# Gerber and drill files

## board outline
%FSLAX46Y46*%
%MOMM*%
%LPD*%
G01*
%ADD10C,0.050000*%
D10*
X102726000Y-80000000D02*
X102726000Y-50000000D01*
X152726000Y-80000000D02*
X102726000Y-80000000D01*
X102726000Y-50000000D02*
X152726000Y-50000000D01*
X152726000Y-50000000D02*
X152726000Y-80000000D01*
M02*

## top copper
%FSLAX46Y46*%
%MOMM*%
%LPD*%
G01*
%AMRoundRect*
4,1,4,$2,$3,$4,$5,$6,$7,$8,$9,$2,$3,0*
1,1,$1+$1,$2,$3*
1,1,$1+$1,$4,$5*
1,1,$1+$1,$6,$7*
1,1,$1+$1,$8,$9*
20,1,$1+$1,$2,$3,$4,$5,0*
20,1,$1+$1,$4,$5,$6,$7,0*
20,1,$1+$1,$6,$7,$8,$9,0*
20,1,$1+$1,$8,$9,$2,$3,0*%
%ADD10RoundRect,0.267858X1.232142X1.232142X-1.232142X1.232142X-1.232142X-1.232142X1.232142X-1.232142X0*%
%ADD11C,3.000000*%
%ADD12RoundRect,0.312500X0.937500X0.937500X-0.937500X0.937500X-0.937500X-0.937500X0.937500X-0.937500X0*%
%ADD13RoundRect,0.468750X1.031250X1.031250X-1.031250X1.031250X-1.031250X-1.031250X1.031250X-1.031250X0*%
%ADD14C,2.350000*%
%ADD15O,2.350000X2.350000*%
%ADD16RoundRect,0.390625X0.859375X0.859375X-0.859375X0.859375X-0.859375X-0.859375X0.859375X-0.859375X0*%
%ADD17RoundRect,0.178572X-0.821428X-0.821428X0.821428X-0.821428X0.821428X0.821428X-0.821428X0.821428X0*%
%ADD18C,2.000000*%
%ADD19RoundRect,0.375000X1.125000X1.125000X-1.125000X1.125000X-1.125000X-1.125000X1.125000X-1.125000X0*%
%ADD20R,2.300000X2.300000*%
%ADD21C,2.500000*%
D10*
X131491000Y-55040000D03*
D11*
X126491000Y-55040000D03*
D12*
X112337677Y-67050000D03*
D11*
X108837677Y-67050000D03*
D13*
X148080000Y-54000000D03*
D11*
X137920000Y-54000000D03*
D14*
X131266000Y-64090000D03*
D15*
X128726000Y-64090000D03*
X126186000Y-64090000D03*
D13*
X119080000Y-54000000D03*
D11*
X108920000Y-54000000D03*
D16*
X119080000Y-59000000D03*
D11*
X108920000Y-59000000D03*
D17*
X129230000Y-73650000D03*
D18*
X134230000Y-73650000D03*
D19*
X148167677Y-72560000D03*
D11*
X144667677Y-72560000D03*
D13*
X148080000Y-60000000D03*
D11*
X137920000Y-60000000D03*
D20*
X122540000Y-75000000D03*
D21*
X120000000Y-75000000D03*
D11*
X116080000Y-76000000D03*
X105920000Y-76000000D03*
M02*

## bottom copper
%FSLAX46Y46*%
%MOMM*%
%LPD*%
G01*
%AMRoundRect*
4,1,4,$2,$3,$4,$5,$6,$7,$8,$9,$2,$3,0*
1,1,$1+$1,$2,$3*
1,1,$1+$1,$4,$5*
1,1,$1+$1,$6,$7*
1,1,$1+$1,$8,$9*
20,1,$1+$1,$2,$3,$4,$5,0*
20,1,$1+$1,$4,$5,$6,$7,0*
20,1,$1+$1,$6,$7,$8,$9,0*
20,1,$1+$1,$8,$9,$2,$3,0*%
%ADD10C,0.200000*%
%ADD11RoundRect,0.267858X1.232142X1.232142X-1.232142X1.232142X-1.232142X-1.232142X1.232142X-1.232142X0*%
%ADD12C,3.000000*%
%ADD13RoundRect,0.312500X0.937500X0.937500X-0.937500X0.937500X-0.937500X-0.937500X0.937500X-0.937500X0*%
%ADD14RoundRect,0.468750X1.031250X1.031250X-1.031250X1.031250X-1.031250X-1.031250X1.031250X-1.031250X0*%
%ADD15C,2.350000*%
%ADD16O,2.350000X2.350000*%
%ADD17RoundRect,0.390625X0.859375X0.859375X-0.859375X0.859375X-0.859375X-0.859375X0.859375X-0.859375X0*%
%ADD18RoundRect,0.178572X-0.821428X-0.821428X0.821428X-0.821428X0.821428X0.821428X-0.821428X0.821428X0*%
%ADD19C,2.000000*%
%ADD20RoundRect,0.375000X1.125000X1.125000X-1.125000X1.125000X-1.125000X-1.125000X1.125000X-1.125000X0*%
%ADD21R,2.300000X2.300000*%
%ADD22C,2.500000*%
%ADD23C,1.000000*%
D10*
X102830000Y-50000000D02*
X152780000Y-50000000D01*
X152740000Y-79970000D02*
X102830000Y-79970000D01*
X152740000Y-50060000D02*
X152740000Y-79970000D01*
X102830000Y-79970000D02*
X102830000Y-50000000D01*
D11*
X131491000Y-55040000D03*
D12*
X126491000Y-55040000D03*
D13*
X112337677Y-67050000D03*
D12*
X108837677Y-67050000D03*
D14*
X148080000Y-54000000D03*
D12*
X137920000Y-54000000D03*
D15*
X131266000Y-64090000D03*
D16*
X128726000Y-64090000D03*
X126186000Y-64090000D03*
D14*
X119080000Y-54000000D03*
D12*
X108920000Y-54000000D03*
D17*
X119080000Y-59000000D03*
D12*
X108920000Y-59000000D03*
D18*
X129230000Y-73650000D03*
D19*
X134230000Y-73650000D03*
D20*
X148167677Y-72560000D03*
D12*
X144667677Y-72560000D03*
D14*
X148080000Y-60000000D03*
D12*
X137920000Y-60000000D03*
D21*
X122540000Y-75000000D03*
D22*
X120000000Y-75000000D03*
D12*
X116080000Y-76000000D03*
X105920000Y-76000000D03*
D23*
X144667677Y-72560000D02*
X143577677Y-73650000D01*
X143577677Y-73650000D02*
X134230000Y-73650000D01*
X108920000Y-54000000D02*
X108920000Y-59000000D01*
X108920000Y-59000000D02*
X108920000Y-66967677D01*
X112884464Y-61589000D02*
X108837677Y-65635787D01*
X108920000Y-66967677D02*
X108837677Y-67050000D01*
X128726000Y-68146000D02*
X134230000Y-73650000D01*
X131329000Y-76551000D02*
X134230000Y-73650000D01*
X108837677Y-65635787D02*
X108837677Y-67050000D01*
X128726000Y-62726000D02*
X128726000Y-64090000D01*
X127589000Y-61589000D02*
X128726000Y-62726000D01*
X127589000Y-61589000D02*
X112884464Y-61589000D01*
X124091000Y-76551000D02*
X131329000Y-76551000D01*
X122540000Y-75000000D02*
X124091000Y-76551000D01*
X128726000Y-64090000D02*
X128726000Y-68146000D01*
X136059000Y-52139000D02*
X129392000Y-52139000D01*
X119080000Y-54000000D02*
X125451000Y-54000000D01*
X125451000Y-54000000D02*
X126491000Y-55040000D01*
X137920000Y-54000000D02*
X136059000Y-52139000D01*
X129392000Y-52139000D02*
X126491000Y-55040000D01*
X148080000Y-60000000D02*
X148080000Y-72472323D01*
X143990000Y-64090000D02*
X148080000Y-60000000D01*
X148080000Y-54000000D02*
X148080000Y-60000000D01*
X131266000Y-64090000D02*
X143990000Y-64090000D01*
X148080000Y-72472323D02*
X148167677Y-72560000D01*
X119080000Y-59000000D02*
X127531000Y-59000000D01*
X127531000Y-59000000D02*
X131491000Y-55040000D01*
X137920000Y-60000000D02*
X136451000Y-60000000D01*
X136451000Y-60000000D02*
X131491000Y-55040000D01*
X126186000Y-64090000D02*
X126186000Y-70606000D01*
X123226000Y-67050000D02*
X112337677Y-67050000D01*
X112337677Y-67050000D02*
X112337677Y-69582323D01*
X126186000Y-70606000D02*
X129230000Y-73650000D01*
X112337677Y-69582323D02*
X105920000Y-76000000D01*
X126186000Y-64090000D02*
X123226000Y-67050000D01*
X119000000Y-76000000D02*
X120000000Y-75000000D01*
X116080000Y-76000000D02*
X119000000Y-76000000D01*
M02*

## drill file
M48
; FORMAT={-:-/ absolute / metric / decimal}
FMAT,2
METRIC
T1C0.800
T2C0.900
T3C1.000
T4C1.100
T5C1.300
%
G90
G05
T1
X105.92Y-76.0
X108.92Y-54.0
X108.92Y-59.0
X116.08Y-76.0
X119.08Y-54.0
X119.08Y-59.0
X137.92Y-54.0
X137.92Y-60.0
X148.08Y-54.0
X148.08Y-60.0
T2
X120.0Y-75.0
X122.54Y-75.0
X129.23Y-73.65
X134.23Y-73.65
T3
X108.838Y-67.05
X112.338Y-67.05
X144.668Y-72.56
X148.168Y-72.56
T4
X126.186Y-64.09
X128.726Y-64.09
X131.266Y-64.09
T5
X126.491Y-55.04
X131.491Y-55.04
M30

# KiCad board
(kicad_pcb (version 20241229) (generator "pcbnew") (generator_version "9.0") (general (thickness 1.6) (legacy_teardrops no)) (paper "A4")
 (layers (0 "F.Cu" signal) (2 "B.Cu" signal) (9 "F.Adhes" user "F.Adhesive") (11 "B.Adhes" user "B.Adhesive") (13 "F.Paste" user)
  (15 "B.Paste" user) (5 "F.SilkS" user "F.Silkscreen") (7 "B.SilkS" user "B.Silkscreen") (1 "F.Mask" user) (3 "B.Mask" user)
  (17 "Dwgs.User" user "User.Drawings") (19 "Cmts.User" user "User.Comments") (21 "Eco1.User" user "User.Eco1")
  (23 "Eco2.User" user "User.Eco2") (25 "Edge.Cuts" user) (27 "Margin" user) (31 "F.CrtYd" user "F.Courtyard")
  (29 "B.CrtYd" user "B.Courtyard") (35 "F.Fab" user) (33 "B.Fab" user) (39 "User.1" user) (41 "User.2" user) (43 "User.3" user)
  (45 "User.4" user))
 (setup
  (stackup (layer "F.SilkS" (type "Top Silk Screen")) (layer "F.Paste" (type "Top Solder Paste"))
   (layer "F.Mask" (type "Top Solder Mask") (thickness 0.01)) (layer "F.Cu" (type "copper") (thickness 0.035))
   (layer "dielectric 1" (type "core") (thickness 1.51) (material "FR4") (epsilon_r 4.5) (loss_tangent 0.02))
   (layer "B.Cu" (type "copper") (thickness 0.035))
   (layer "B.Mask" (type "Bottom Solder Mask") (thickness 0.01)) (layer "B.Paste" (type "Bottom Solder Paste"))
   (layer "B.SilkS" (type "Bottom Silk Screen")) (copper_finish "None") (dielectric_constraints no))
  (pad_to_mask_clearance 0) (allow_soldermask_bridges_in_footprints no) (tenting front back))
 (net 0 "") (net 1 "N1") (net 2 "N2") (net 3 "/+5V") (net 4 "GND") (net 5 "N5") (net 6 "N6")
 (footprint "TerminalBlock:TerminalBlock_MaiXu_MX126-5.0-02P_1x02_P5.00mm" (layer "F.Cu") (at 131.491 55.04 180)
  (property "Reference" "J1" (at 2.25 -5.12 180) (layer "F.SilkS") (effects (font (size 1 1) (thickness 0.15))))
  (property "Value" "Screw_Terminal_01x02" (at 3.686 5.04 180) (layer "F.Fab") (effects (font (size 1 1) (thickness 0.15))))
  (pad "1" thru_hole roundrect (at 0 0 180) (size 3 3) (drill 1.3) (layers "*.Cu" "*.Mask") (remove_unused_layers no)
   (roundrect_rratio 0.089286) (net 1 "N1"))
  (pad "2" thru_hole circle (at 5 0 180) (size 3 3) (drill 1.3) (layers "*.Cu" "*.Mask") (remove_unused_layers no) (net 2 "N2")))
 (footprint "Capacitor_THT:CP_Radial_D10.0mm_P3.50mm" (layer "F.Cu") (at 112.337677 67.05 180)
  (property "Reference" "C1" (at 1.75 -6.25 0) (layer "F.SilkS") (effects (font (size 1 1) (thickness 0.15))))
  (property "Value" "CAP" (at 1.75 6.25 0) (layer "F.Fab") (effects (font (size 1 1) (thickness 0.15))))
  (pad "1" thru_hole roundrect (at 0 0 180) (size 2.5 2.5) (drill 1) (layers "*.Cu" "*.Mask") (remove_unused_layers no)
   (roundrect_rratio 0.125) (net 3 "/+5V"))
  (pad "2" thru_hole circle (at 3.5 0 180) (size 3 3) (drill 1) (layers "*.Cu" "*.Mask") (remove_unused_layers no) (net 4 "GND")))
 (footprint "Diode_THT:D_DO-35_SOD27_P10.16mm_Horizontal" (layer "F.Cu") (at 148.08 54 180)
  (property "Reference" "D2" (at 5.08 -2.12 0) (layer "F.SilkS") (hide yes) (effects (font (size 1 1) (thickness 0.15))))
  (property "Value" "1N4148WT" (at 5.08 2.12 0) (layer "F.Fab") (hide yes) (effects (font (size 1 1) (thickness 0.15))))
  (pad "1" thru_hole roundrect (at 0 0 180) (size 3 3) (drill 0.8) (layers "*.Cu" "*.Mask") (remove_unused_layers no)
   (roundrect_rratio 0.15625) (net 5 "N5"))
  (pad "2" thru_hole circle (at 10.16 0 180) (size 3 3) (drill 0.8) (layers "*.Cu" "*.Mask") (remove_unused_layers no) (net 2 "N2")))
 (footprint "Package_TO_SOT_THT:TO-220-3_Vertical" (layer "F.Cu") (at 131.266 64.09 180)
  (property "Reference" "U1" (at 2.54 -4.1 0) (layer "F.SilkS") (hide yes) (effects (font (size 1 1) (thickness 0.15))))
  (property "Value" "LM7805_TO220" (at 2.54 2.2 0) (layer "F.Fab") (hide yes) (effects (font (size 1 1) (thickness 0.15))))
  (pad "1" thru_hole circle (at 0 0 180) (size 2.35 2.35) (drill 1.1) (layers "*.Cu" "*.Mask") (remove_unused_layers no) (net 5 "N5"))
  (pad "2" thru_hole oval (at 2.54 0 180) (size 2.35 2.35) (drill 1.1) (layers "*.Cu" "*.Mask") (remove_unused_layers no) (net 4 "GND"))
  (pad "3" thru_hole oval (at 5.08 0 180) (size 2.35 2.35) (drill 1.1) (layers "*.Cu" "*.Mask") (remove_unused_layers no) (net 3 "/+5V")))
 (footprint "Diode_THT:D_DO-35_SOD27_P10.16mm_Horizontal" (layer "F.Cu") (at 119.08 54 180)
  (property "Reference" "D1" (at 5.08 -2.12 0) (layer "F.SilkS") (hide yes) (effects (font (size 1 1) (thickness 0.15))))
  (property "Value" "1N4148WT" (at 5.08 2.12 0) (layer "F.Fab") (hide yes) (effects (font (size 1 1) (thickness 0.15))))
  (pad "1" thru_hole roundrect (at 0 0 180) (size 3 3) (drill 0.8) (layers "*.Cu" "*.Mask") (remove_unused_layers no)
   (roundrect_rratio 0.15625) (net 2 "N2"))
  (pad "2" thru_hole circle (at 10.16 0 180) (size 3 3) (drill 0.8) (layers "*.Cu" "*.Mask") (remove_unused_layers no) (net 4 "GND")))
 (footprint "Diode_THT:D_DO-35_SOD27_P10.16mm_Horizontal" (layer "F.Cu") (at 119.08 59 180)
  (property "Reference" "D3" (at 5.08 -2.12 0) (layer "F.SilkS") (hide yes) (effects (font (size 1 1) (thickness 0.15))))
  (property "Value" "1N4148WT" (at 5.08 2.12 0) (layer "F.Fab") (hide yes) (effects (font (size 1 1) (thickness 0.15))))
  (pad "1" thru_hole roundrect (at 0 0 180) (size 2.5 2.5) (drill 0.8) (layers "*.Cu" "*.Mask") (remove_unused_layers no)
   (roundrect_rratio 0.15625) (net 1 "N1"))
  (pad "2" thru_hole circle (at 10.16 0 180) (size 3 3) (drill 0.8) (layers "*.Cu" "*.Mask") (remove_unused_layers no) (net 4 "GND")))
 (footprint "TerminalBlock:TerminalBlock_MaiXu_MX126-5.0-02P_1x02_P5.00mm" (layer "F.Cu") (at 129.23 73.65)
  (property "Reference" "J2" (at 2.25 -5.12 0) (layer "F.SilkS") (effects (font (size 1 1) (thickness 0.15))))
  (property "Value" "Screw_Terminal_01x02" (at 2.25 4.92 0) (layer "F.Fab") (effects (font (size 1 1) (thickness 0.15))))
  (pad "1" thru_hole roundrect (at 0 0) (size 2 2) (drill 0.9) (layers "*.Cu" "*.Mask") (remove_unused_layers no)
   (roundrect_rratio 0.089286) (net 3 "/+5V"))
  (pad "2" thru_hole circle (at 5 0) (size 2 2) (drill 0.9) (layers "*.Cu" "*.Mask") (remove_unused_layers no) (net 4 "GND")))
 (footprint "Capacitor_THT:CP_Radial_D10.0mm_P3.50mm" (layer "F.Cu") (at 148.167677 72.56 180)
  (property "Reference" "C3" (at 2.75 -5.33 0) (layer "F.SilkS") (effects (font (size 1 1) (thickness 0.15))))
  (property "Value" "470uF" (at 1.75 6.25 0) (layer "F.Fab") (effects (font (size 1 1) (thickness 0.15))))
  (pad "1" thru_hole roundrect (at 0 0 180) (size 3 3) (drill 1) (layers "*.Cu" "*.Mask") (remove_unused_layers no) (roundrect_rratio 0.125)
   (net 5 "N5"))
  (pad "2" thru_hole circle (at 3.5 0 180) (size 3 3) (drill 1) (layers "*.Cu" "*.Mask") (remove_unused_layers no) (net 4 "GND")))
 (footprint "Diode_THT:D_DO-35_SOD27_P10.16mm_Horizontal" (layer "F.Cu") (at 148.08 60 180)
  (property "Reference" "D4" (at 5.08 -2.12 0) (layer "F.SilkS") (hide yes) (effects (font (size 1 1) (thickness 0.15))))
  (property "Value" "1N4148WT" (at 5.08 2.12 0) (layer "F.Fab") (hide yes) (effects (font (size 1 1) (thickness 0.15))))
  (pad "1" thru_hole roundrect (at 0 0 180) (size 3 3) (drill 0.8) (layers "*.Cu" "*.Mask") (remove_unused_layers no)
   (roundrect_rratio 0.15625) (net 5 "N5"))
  (pad "2" thru_hole circle (at 10.16 0 180) (size 3 3) (drill 0.8) (layers "*.Cu" "*.Mask") (remove_unused_layers no) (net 1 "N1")))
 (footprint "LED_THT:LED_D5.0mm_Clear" (layer "F.Cu") (at 122.54 75 180)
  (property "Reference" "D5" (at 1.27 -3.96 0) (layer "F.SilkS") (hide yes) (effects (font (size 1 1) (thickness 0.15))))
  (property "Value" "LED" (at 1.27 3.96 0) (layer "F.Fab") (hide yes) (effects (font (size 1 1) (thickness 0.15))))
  (pad "1" thru_hole rect (at 0 0 180) (size 2.3 2.3) (drill 0.9) (layers "*.Cu" "*.Mask") (remove_unused_layers no) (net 4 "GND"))
  (pad "2" thru_hole circle (at 2.54 0 180) (size 2.5 2.5) (drill 0.9) (layers "*.Cu" "*.Mask") (remove_unused_layers no) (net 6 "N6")))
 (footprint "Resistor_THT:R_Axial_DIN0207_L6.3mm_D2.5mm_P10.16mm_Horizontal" (layer "F.Cu") (at 116.08 76 180)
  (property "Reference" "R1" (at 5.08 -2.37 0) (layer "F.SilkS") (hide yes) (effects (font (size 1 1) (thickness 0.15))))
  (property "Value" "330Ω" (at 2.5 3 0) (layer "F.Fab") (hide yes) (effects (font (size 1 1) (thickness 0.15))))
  (pad "1" thru_hole circle (at 0 0 180) (size 3 3) (drill 0.8) (layers "*.Cu" "*.Mask") (remove_unused_layers no) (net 6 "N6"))
  (pad "2" thru_hole circle (at 10.16 0 180) (size 3 3) (drill 0.8) (layers "*.Cu" "*.Mask") (remove_unused_layers no) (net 3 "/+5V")))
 (gr_line (start 102.83 50) (end 152.78 50) (stroke (width 0.2) (type default)) (layer "B.Cu"))
 (gr_line (start 152.74 79.97) (end 102.83 79.97) (stroke (width 0.2) (type default)) (layer "B.Cu"))
 (gr_line (start 152.74 50.06) (end 152.74 79.97) (stroke (width 0.2) (type default)) (layer "B.Cu"))
 (gr_line (start 102.83 79.97) (end 102.83 50) (stroke (width 0.2) (type default)) (layer "B.Cu"))
 (gr_line (start 102.726 80) (end 102.726 50) (stroke (width 0.05) (type default)) (layer "Edge.Cuts"))
 (gr_line (start 152.726 80) (end 102.726 80) (stroke (width 0.05) (type default)) (layer "Edge.Cuts"))
 (gr_line (start 102.726 50) (end 152.726 50) (stroke (width 0.05) (type default)) (layer "Edge.Cuts"))
 (gr_line (start 152.726 50) (end 152.726 80) (stroke (width 0.05) (type default)) (layer "Edge.Cuts"))
 (segment (start 144.667677 72.56) (end 143.577677 73.65) (width 1) (layer "B.Cu") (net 4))
 (segment (start 143.577677 73.65) (end 134.23 73.65) (width 1) (layer "B.Cu") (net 4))
 (segment (start 108.92 54) (end 108.92 59) (width 1) (layer "B.Cu") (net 4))
 (segment (start 108.92 59) (end 108.92 66.967677) (width 1) (layer "B.Cu") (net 4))
 (segment (start 112.884464 61.589) (end 108.837677 65.635787) (width 1) (layer "B.Cu") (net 4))
 (segment (start 108.92 66.967677) (end 108.837677 67.05) (width 1) (layer "B.Cu") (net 4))
 (segment (start 128.726 68.146) (end 134.23 73.65) (width 1) (layer "B.Cu") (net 4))
 (segment (start 131.329 76.551) (end 134.23 73.65) (width 1) (layer "B.Cu") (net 4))
 (segment (start 108.837677 65.635787) (end 108.837677 67.05) (width 1) (layer "B.Cu") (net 4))
 (segment (start 128.726 62.726) (end 128.726 64.09) (width 1) (layer "B.Cu") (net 4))
 (segment (start 127.589 61.589) (end 128.726 62.726) (width 1) (layer "B.Cu") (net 4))
 (segment (start 127.589 61.589) (end 112.884464 61.589) (width 1) (layer "B.Cu") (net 4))
 (segment (start 124.091 76.551) (end 131.329 76.551) (width 1) (layer "B.Cu") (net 4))
 (segment (start 122.54 75) (end 124.091 76.551) (width 1) (layer "B.Cu") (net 4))
 (segment (start 128.726 64.09) (end 128.726 68.146) (width 1) (layer "B.Cu") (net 4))
 (segment (start 136.059 52.139) (end 129.392 52.139) (width 1) (layer "B.Cu") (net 2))
 (segment (start 119.08 54) (end 125.451 54) (width 1) (layer "B.Cu") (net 2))
 (segment (start 125.451 54) (end 126.491 55.04) (width 1) (layer "B.Cu") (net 2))
 (segment (start 137.92 54) (end 136.059 52.139) (width 1) (layer "B.Cu") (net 2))
 (segment (start 129.392 52.139) (end 126.491 55.04) (width 1) (layer "B.Cu") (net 2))
 (segment (start 148.08 60) (end 148.08 72.472323) (width 1) (layer "B.Cu") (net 5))
 (segment (start 143.99 64.09) (end 148.08 60) (width 1) (layer "B.Cu") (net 5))
 (segment (start 148.08 54) (end 148.08 60) (width 1) (layer "B.Cu") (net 5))
 (segment (start 131.266 64.09) (end 143.99 64.09) (width 1) (layer "B.Cu") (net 5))
 (segment (start 148.08 72.472323) (end 148.167677 72.56) (width 1) (layer "B.Cu") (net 5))
 (segment (start 119.08 59) (end 127.531 59) (width 1) (layer "B.Cu") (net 1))
 (segment (start 127.531 59) (end 131.491 55.04) (width 1) (layer "B.Cu") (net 1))
 (segment (start 137.92 60) (end 136.451 60) (width 1) (layer "B.Cu") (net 1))
 (segment (start 136.451 60) (end 131.491 55.04) (width 1) (layer "B.Cu") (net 1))
 (segment (start 126.186 64.09) (end 126.186 70.606) (width 1) (layer "B.Cu") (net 3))
 (segment (start 123.226 67.05) (end 112.337677 67.05) (width 1) (layer "B.Cu") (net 3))
 (segment (start 112.337677 67.05) (end 112.337677 69.582323) (width 1) (layer "B.Cu") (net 3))
 (segment (start 126.186 70.606) (end 129.23 73.65) (width 1) (layer "B.Cu") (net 3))
 (segment (start 112.337677 69.582323) (end 105.92 76) (width 1) (layer "B.Cu") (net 3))
 (segment (start 126.186 64.09) (end 123.226 67.05) (width 1) (layer "B.Cu") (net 3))
 (segment (start 119 76) (end 120 75) (width 1) (layer "B.Cu") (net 6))
 (segment (start 116.08 76) (end 119 76) (width 1) (layer "B.Cu") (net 6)))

